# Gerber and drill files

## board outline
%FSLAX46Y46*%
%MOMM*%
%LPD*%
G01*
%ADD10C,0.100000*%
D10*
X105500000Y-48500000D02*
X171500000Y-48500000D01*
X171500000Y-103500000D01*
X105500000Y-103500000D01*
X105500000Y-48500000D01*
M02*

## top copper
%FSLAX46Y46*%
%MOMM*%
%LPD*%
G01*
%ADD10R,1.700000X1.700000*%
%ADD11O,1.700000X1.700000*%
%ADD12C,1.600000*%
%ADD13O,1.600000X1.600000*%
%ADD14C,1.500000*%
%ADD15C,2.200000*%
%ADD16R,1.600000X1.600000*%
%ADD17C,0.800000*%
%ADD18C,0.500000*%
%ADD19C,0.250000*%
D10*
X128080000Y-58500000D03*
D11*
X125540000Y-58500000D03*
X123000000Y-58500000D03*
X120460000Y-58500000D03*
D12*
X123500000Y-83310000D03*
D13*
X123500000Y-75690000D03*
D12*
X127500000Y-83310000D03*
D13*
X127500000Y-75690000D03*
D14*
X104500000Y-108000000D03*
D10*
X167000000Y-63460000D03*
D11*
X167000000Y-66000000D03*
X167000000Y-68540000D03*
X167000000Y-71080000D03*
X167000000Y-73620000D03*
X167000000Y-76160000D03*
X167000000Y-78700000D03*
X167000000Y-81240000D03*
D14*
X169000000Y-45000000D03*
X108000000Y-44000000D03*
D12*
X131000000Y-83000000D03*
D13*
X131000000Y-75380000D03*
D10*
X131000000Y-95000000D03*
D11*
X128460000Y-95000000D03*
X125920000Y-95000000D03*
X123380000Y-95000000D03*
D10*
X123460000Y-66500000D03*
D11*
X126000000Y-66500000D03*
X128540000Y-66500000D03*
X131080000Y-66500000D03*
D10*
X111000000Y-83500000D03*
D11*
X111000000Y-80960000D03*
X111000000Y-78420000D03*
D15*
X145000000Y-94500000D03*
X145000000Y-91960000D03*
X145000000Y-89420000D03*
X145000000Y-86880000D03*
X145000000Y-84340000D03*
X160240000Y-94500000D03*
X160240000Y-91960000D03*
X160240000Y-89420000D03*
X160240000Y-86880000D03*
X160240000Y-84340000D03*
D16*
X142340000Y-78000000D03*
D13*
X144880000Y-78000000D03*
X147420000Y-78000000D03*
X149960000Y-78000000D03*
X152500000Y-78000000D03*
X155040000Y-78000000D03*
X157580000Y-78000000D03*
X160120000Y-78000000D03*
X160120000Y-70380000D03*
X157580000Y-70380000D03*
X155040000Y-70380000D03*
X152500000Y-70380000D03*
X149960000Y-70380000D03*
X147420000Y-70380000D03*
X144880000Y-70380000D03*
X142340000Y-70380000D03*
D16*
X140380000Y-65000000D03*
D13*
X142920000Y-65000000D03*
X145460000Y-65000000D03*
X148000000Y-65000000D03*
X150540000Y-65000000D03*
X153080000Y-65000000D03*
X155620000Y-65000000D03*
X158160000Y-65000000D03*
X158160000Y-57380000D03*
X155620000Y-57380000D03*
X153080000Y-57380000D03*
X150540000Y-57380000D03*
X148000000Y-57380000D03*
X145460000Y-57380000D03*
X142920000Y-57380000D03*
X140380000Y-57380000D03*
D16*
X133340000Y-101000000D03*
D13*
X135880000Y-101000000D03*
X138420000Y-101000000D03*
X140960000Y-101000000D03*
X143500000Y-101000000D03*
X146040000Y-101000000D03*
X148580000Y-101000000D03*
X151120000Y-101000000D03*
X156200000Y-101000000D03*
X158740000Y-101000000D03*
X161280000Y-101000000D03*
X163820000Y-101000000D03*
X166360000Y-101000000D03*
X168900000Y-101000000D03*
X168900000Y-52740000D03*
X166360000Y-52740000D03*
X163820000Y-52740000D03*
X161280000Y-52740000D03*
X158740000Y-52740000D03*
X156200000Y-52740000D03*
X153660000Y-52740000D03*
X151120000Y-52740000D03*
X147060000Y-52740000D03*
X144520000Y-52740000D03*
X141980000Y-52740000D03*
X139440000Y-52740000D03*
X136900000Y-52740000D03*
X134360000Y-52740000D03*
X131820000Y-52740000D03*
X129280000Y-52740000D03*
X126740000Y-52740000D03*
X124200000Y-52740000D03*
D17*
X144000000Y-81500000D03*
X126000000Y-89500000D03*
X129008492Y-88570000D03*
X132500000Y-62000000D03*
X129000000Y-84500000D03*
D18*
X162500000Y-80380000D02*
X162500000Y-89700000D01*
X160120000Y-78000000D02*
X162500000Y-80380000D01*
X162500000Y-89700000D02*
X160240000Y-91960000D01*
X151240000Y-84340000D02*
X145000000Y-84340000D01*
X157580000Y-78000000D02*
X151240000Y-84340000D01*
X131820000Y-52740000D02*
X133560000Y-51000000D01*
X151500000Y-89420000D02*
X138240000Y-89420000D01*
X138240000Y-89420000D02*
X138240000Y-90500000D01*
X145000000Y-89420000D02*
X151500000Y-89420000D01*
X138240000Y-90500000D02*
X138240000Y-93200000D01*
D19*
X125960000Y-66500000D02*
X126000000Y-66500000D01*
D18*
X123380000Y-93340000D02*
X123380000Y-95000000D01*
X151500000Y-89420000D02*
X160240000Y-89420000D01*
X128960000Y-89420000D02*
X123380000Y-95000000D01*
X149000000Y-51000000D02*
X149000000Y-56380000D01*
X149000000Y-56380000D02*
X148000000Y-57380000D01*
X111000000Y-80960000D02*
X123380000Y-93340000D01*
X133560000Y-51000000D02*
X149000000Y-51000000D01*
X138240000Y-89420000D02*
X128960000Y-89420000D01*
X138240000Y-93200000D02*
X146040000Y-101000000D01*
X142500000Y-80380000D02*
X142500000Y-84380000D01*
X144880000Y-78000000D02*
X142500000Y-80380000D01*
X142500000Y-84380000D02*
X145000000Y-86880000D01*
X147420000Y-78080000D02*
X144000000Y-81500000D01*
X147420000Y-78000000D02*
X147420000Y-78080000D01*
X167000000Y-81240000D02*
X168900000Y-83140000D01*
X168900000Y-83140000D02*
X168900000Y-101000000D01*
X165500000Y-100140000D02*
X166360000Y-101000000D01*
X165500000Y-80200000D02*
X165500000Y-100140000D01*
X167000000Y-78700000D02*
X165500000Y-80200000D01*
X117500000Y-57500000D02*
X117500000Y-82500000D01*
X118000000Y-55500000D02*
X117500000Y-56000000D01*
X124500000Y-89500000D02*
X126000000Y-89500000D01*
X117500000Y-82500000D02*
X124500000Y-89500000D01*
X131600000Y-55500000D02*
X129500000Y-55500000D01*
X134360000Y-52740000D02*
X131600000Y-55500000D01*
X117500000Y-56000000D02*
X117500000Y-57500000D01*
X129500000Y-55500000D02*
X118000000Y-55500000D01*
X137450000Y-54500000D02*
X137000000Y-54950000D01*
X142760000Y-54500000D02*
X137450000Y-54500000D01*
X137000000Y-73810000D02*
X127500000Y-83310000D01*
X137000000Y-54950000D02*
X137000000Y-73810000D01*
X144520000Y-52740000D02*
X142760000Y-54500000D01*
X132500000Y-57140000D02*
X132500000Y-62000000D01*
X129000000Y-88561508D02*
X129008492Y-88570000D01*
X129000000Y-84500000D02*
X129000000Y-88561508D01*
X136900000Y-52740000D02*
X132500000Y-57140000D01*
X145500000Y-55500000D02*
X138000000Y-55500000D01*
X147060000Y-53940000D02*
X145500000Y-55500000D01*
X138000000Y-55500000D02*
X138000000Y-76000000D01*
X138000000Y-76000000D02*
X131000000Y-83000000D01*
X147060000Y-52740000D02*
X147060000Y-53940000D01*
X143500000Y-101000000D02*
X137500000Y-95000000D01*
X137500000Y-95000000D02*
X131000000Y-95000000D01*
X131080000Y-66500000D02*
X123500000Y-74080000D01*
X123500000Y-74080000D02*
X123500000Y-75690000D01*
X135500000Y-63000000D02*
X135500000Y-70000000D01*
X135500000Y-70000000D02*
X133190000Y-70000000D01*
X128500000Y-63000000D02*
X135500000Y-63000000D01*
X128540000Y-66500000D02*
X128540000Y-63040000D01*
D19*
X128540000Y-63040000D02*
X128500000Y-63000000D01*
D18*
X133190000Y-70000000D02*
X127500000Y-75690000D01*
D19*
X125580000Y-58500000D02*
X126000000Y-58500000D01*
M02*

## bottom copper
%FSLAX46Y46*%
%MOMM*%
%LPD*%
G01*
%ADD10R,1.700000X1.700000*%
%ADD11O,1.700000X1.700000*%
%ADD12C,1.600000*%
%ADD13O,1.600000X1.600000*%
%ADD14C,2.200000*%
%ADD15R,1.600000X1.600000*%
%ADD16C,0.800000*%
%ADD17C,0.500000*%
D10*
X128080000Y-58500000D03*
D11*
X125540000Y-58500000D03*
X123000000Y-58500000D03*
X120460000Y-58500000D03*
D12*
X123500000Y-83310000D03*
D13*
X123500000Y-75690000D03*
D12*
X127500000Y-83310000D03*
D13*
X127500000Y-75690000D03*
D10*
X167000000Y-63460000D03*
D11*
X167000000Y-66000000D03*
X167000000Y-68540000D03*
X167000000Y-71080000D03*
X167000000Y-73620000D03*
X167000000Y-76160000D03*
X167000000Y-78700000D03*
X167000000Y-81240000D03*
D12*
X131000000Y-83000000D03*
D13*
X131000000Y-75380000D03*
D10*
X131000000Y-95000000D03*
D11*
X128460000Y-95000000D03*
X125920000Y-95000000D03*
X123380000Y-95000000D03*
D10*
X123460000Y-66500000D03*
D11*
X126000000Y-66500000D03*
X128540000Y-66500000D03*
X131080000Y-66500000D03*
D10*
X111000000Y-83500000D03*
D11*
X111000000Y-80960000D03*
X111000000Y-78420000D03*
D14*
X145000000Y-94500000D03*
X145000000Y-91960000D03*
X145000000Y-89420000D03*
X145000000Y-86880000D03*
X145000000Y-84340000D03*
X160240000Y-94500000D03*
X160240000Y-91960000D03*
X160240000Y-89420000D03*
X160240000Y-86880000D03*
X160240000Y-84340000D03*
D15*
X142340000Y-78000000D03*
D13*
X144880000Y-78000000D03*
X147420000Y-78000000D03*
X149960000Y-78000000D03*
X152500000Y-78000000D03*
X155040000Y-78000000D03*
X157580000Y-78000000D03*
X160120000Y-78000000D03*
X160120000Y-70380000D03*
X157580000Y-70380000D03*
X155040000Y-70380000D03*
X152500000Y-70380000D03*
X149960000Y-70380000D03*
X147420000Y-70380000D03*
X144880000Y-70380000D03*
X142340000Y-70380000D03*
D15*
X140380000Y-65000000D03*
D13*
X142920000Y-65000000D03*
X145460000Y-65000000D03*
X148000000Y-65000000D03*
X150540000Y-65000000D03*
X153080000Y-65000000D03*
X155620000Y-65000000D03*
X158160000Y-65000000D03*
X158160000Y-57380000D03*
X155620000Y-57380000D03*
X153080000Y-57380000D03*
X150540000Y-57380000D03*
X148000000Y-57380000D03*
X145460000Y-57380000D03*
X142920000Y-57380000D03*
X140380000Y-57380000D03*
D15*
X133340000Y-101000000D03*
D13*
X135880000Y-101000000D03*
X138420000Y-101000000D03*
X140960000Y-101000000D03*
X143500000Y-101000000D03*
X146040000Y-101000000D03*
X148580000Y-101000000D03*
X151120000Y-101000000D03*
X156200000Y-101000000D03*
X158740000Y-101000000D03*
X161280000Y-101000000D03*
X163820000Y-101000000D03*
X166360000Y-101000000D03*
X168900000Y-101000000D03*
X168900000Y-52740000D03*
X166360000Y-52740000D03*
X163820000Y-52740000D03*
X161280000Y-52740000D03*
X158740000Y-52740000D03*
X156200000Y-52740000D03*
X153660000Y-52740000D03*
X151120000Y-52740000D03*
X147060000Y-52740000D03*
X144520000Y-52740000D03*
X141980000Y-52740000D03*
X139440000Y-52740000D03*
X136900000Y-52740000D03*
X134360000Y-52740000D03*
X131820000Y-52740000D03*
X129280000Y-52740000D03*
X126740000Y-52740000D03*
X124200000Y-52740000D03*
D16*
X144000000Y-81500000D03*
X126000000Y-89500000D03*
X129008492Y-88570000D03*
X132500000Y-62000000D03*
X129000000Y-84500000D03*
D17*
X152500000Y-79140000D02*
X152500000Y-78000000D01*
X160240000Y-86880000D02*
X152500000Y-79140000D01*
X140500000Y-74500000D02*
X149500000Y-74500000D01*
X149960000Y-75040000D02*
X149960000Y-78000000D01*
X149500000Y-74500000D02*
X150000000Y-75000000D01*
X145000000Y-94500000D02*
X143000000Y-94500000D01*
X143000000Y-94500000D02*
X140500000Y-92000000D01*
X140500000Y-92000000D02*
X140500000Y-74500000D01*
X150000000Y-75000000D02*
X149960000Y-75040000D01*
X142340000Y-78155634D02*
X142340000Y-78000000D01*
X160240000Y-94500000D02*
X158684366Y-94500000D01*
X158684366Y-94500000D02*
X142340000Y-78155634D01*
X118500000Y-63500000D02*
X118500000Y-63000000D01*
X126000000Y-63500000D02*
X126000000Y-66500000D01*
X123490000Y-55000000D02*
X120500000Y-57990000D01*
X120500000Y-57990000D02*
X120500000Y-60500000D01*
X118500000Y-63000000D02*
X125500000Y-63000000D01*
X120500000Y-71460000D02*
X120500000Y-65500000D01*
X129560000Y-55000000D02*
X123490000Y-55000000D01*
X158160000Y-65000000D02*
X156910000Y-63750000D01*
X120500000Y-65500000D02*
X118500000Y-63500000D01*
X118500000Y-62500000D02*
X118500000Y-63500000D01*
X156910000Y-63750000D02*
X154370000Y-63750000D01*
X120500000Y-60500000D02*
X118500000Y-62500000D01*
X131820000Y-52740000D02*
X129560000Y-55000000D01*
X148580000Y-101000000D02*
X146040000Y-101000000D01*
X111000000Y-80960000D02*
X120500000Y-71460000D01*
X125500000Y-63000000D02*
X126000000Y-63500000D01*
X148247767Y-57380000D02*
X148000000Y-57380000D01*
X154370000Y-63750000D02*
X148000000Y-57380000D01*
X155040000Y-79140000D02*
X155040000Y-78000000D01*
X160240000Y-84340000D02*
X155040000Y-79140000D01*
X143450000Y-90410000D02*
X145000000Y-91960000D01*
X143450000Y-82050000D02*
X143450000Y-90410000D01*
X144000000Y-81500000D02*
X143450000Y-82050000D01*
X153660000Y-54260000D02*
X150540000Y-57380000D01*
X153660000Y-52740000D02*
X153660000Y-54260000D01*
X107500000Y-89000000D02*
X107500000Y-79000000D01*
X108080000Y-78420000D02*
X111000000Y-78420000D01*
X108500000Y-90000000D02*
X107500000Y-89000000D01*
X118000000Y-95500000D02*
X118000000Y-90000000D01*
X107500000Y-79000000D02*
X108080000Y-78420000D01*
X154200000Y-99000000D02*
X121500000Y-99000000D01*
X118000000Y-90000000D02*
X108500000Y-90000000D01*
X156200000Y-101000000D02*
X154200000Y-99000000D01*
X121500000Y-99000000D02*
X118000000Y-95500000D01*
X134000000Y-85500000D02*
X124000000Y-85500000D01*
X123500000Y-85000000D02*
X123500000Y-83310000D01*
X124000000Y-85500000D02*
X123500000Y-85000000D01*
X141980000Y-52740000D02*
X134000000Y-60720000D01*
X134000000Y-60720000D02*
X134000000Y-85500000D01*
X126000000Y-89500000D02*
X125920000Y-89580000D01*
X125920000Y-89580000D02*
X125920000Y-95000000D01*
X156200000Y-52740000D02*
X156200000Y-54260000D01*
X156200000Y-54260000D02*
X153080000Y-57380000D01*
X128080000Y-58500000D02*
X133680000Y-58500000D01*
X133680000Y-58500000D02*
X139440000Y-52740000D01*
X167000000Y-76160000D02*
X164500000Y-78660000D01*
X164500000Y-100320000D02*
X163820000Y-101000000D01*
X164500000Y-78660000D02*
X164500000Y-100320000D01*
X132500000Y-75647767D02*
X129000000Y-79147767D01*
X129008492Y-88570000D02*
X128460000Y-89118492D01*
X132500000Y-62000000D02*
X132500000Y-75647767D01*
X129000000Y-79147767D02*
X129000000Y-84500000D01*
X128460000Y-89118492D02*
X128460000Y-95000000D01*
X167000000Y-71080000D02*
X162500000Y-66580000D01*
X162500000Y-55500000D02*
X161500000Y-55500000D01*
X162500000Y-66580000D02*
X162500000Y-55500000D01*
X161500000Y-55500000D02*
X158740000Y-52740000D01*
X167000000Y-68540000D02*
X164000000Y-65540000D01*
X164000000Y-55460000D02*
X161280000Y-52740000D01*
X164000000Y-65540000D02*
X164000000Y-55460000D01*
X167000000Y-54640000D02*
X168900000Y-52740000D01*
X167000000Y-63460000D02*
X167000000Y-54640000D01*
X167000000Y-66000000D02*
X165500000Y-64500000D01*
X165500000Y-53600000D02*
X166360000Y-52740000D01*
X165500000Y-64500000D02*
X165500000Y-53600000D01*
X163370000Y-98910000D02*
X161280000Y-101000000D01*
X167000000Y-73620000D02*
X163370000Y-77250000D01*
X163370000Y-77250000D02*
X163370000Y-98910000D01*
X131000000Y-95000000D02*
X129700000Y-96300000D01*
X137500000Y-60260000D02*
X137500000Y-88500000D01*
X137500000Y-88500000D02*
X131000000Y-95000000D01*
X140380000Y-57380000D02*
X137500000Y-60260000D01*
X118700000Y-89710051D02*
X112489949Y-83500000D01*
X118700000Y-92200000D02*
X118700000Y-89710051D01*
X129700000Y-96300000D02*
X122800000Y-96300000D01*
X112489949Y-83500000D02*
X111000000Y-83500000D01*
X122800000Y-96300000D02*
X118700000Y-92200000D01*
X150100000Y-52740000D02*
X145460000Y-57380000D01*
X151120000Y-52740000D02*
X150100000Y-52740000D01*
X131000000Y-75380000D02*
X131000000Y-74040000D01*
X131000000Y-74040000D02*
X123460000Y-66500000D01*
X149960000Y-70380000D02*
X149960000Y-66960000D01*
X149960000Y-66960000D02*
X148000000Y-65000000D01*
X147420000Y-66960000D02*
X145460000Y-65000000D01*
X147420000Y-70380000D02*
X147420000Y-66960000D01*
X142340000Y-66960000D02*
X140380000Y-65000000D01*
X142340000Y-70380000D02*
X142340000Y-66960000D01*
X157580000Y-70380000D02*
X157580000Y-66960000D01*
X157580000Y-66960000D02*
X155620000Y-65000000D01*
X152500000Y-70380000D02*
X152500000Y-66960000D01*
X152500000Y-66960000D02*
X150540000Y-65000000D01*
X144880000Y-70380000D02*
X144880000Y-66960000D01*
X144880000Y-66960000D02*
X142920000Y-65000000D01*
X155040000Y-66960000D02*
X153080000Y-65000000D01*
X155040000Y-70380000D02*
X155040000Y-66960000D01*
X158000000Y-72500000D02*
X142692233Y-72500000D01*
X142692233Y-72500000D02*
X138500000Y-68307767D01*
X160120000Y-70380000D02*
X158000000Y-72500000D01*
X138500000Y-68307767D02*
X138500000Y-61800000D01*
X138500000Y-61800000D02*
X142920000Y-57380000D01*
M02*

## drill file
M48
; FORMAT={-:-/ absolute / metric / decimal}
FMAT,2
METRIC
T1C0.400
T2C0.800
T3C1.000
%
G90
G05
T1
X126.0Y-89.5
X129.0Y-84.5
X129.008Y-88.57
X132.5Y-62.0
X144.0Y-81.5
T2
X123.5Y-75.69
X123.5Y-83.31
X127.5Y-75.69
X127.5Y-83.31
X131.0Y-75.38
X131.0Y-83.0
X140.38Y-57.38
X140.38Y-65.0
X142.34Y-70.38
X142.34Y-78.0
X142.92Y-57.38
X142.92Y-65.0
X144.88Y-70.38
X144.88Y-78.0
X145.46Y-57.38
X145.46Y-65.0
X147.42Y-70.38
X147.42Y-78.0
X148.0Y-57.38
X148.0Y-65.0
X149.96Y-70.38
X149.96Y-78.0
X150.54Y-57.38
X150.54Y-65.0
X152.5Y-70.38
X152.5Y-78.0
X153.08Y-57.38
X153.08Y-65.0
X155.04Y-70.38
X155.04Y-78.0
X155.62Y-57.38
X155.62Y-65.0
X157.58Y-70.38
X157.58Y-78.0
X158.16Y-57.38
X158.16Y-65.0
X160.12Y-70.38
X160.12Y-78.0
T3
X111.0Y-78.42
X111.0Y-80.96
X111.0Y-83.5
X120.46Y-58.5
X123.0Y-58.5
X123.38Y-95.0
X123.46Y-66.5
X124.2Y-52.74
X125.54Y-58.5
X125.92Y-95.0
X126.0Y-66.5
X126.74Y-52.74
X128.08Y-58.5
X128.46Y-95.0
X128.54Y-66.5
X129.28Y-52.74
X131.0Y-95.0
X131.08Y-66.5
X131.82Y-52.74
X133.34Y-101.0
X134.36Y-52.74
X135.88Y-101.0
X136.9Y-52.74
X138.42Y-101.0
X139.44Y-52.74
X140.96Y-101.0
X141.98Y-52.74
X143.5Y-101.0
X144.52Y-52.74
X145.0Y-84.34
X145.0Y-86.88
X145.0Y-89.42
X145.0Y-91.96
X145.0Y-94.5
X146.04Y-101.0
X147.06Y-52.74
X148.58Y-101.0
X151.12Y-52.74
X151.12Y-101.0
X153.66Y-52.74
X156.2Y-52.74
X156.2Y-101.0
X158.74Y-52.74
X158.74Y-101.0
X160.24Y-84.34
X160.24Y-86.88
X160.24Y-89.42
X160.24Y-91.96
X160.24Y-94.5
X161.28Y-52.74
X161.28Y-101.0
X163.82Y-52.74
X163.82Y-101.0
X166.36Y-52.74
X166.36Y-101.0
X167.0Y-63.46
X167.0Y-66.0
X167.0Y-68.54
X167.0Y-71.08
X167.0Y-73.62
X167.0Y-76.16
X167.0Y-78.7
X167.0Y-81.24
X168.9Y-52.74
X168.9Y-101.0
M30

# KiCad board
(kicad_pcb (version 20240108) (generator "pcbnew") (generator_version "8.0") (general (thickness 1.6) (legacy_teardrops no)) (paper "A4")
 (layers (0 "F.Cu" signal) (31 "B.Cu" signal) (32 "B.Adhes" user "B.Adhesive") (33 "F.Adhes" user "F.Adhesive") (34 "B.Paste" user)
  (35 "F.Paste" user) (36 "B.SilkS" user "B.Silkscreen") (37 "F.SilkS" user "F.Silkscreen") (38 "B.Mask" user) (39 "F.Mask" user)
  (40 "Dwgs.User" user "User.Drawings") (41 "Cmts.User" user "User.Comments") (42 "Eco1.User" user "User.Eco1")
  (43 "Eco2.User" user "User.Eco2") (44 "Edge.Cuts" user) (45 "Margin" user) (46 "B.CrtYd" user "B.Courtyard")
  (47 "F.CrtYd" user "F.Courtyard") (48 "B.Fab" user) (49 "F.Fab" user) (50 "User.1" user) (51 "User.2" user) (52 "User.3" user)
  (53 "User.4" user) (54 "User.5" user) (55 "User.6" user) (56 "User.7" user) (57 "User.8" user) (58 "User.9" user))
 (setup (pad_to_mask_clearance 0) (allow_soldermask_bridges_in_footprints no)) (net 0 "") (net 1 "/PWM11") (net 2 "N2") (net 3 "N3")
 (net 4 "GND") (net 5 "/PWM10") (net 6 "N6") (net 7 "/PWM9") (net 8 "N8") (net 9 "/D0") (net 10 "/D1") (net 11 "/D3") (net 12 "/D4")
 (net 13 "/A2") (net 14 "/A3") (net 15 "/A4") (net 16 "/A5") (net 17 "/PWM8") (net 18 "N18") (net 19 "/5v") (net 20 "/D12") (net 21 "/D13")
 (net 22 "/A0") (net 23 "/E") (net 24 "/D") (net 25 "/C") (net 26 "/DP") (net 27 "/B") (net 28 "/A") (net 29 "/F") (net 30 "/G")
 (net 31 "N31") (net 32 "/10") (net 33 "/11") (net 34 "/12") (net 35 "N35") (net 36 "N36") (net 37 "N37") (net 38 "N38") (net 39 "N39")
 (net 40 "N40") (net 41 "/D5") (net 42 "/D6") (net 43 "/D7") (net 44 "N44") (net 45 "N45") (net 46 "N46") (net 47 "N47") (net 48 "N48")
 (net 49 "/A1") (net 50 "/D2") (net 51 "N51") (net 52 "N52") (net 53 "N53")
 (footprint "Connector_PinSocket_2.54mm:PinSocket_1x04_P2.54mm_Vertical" (layer "F.Cu") (at 128.08 58.5 -90)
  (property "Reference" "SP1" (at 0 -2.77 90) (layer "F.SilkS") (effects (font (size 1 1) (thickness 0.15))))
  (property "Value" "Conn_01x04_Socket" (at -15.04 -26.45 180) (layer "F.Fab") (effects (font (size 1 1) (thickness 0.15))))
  (pad "1" thru_hole rect (at 0 0 270) (size 1.7 1.7) (drill 1) (layers "*.Cu" "*.Mask") (remove_unused_layers no) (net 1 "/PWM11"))
  (pad "2" thru_hole oval (at 0 2.54 270) (size 1.7 1.7) (drill 1) (layers "*.Cu" "*.Mask") (remove_unused_layers no) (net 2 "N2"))
  (pad "3" thru_hole oval (at 0 5.08 270) (size 1.7 1.7) (drill 1) (layers "*.Cu" "*.Mask") (remove_unused_layers no) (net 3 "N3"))
  (pad "4" thru_hole oval (at 0 7.62 270) (size 1.7 1.7) (drill 1) (layers "*.Cu" "*.Mask") (remove_unused_layers no) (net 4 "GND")))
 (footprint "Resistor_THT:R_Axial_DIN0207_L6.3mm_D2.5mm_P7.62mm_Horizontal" (layer "F.Cu") (at 123.5 83.31 90)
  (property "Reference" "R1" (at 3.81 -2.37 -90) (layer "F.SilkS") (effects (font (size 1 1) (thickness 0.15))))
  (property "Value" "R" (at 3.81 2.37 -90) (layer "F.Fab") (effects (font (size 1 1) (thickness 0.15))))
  (pad "1" thru_hole circle (at 0 0 90) (size 1.6 1.6) (drill 0.8) (layers "*.Cu" "*.Mask") (remove_unused_layers no) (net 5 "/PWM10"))
  (pad "2" thru_hole oval (at 7.62 0 90) (size 1.6 1.6) (drill 0.8) (layers "*.Cu" "*.Mask") (remove_unused_layers no) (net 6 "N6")))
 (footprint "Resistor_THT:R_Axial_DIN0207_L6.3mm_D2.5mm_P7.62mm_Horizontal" (layer "F.Cu") (at 127.5 83.31 90)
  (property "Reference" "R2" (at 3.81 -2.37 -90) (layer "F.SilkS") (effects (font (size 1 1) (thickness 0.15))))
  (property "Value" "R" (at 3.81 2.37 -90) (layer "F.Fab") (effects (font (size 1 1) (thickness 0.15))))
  (pad "1" thru_hole circle (at 0 0 90) (size 1.6 1.6) (drill 0.8) (layers "*.Cu" "*.Mask") (remove_unused_layers no) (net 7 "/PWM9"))
  (pad "2" thru_hole oval (at 7.62 0 90) (size 1.6 1.6) (drill 0.8) (layers "*.Cu" "*.Mask") (remove_unused_layers no) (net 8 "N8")))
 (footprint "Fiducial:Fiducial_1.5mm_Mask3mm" (layer "F.Cu") (at 104.5 108)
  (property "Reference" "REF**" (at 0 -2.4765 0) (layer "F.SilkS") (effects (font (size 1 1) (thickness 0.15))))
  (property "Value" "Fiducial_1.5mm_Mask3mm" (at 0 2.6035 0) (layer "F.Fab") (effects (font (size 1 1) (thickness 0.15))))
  (pad "" smd circle (at 0 0) (size 1.5 1.5) (layers "F.Cu" "F.Mask") (solder_mask_margin 0.75) (clearance 0.75)))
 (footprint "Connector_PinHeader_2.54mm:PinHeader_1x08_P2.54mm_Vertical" (layer "F.Cu") (at 167 63.46)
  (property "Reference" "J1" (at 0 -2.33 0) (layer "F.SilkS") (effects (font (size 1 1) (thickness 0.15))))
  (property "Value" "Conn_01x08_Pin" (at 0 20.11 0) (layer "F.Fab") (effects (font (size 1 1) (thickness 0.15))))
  (pad "1" thru_hole rect (at 0 0) (size 1.7 1.7) (drill 1) (layers "*.Cu" "*.Mask") (remove_unused_layers no) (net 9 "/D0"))
  (pad "2" thru_hole oval (at 0 2.54) (size 1.7 1.7) (drill 1) (layers "*.Cu" "*.Mask") (remove_unused_layers no) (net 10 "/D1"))
  (pad "3" thru_hole oval (at 0 5.08) (size 1.7 1.7) (drill 1) (layers "*.Cu" "*.Mask") (remove_unused_layers no) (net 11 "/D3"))
  (pad "4" thru_hole oval (at 0 7.62) (size 1.7 1.7) (drill 1) (layers "*.Cu" "*.Mask") (remove_unused_layers no) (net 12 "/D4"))
  (pad "5" thru_hole oval (at 0 10.16) (size 1.7 1.7) (drill 1) (layers "*.Cu" "*.Mask") (remove_unused_layers no) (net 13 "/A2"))
  (pad "6" thru_hole oval (at 0 12.7) (size 1.7 1.7) (drill 1) (layers "*.Cu" "*.Mask") (remove_unused_layers no) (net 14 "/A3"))
  (pad "7" thru_hole oval (at 0 15.24) (size 1.7 1.7) (drill 1) (layers "*.Cu" "*.Mask") (remove_unused_layers no) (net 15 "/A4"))
  (pad "8" thru_hole oval (at 0 17.78) (size 1.7 1.7) (drill 1) (layers "*.Cu" "*.Mask") (remove_unused_layers no) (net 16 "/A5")))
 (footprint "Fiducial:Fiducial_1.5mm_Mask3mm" (layer "F.Cu") (at 169 45)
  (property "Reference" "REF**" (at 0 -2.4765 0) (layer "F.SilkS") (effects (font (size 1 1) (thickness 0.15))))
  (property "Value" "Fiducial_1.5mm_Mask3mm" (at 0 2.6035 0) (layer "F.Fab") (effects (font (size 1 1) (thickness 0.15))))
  (pad "" smd circle (at 0 0) (size 1.5 1.5) (layers "F.Cu" "F.Mask") (solder_mask_margin 0.75) (clearance 0.75)))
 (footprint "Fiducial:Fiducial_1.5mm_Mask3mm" (layer "F.Cu") (at 108 44)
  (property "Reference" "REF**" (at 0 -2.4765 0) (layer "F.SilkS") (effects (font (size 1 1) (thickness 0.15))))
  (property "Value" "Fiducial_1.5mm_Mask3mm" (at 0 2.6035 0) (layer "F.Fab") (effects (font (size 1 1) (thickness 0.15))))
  (pad "" smd circle (at 0 0) (size 1.5 1.5) (layers "F.Cu" "F.Mask") (solder_mask_margin 0.75) (clearance 0.75)))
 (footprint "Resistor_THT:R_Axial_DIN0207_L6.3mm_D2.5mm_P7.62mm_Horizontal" (layer "F.Cu") (at 131 83 90)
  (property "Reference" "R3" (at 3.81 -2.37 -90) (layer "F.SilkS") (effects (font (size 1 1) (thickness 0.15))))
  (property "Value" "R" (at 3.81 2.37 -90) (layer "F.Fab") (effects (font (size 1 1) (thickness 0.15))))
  (pad "1" thru_hole circle (at 0 0 90) (size 1.6 1.6) (drill 0.8) (layers "*.Cu" "*.Mask") (remove_unused_layers no) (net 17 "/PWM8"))
  (pad "2" thru_hole oval (at 7.62 0 90) (size 1.6 1.6) (drill 0.8) (layers "*.Cu" "*.Mask") (remove_unused_layers no) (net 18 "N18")))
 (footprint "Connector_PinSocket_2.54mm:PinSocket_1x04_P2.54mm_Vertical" (layer "F.Cu") (at 131 95 -90)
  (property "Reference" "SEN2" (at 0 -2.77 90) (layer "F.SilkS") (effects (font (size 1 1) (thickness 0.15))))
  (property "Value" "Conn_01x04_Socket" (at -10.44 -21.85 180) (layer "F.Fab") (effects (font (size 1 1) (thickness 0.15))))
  (pad "1" thru_hole rect (at 0 0 270) (size 1.7 1.7) (drill 1) (layers "*.Cu" "*.Mask") (remove_unused_layers no) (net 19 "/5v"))
  (pad "2" thru_hole oval (at 0 2.54 270) (size 1.7 1.7) (drill 1) (layers "*.Cu" "*.Mask") (remove_unused_layers no) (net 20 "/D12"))
  (pad "3" thru_hole oval (at 0 5.08 270) (size 1.7 1.7) (drill 1) (layers "*.Cu" "*.Mask") (remove_unused_layers no) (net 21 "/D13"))
  (pad "4" thru_hole oval (at 0 7.62 270) (size 1.7 1.7) (drill 1) (layers "*.Cu" "*.Mask") (remove_unused_layers no) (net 4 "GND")))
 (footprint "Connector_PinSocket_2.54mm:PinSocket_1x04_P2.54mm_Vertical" (layer "F.Cu") (at 123.46 66.5 90)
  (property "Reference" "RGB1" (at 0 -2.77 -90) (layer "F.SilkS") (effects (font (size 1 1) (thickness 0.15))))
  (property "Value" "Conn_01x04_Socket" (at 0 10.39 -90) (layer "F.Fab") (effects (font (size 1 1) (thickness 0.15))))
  (pad "1" thru_hole rect (at 0 0 90) (size 1.7 1.7) (drill 1) (layers "*.Cu" "*.Mask") (remove_unused_layers no) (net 18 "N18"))
  (pad "2" thru_hole oval (at 0 2.54 90) (size 1.7 1.7) (drill 1) (layers "*.Cu" "*.Mask") (remove_unused_layers no) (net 4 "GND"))
  (pad "3" thru_hole oval (at 0 5.08 90) (size 1.7 1.7) (drill 1) (layers "*.Cu" "*.Mask") (remove_unused_layers no) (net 8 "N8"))
  (pad "4" thru_hole oval (at 0 7.62 90) (size 1.7 1.7) (drill 1) (layers "*.Cu" "*.Mask") (remove_unused_layers no) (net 6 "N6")))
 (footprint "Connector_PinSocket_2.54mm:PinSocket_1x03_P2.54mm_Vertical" (layer "F.Cu") (at 111 83.5 180)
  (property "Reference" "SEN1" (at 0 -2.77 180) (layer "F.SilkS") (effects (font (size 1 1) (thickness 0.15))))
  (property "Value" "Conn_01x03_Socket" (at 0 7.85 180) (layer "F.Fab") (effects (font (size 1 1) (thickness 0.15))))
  (pad "1" thru_hole rect (at 0 0 180) (size 1.7 1.7) (drill 1) (layers "*.Cu" "*.Mask") (remove_unused_layers no) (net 19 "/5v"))
  (pad "2" thru_hole oval (at 0 2.54 180) (size 1.7 1.7) (drill 1) (layers "*.Cu" "*.Mask") (remove_unused_layers no) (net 4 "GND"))
  (pad "3" thru_hole oval (at 0 5.08 180) (size 1.7 1.7) (drill 1) (layers "*.Cu" "*.Mask") (remove_unused_layers no) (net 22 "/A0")))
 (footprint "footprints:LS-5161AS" (layer "F.Cu") (at 145 94.5 90)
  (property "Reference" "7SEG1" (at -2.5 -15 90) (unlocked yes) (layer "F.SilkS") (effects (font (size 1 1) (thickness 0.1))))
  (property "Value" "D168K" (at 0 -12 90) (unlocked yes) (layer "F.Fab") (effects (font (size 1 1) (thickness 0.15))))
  (pad "1" thru_hole circle (at 0 0 90) (size 2.2 2.2) (drill 1) (layers "*.Cu" "*.Mask") (remove_unused_layers no) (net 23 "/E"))
  (pad "2" thru_hole circle (at 2.54 0 90) (size 2.2 2.2) (drill 1) (layers "*.Cu" "*.Mask") (remove_unused_layers no) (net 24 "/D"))
  (pad "3" thru_hole circle (at 5.08 0 90) (size 2.2 2.2) (drill 1) (layers "*.Cu" "*.Mask") (remove_unused_layers no) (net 4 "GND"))
  (pad "4" thru_hole circle (at 7.62 0 90) (size 2.2 2.2) (drill 1) (layers "*.Cu" "*.Mask") (remove_unused_layers no) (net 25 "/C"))
  (pad "5" thru_hole circle (at 10.16 0 90) (size 2.2 2.2) (drill 1) (layers "*.Cu" "*.Mask") (remove_unused_layers no) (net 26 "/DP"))
  (pad "6" thru_hole circle (at 0 15.24 90) (size 2.2 2.2) (drill 1) (layers "*.Cu" "*.Mask") (remove_unused_layers no) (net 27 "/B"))
  (pad "7" thru_hole circle (at 2.54 15.24 90) (size 2.2 2.2) (drill 1) (layers "*.Cu" "*.Mask") (remove_unused_layers no) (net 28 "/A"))
  (pad "8" thru_hole circle (at 5.08 15.24 90) (size 2.2 2.2) (drill 1) (layers "*.Cu" "*.Mask") (remove_unused_layers no) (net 4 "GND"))
  (pad "9" thru_hole circle (at 7.62 15.24 90) (size 2.2 2.2) (drill 1) (layers "*.Cu" "*.Mask") (remove_unused_layers no) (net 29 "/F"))
  (pad "10" thru_hole circle (at 10.16 15.24 90) (size 2.2 2.2) (drill 1) (layers "*.Cu" "*.Mask") (remove_unused_layers no) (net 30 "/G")))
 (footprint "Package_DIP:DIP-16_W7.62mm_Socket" (layer "F.Cu") (at 142.34 78 90)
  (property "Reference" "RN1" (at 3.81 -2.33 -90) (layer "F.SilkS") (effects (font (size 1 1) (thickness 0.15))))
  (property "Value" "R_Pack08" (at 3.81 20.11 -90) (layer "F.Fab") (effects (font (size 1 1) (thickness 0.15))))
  (pad "1" thru_hole rect (at 0 0 90) (size 1.6 1.6) (drill 0.8) (layers "*.Cu" "*.Mask") (remove_unused_layers no) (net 27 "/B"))
  (pad "2" thru_hole oval (at 0 2.54 90) (size 1.6 1.6) (drill 0.8) (layers "*.Cu" "*.Mask") (remove_unused_layers no) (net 25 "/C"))
  (pad "3" thru_hole oval (at 0 5.08 90) (size 1.6 1.6) (drill 0.8) (layers "*.Cu" "*.Mask") (remove_unused_layers no) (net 24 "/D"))
  (pad "4" thru_hole oval (at 0 7.62 90) (size 1.6 1.6) (drill 0.8) (layers "*.Cu" "*.Mask") (remove_unused_layers no) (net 23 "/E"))
  (pad "5" thru_hole oval (at 0 10.16 90) (size 1.6 1.6) (drill 0.8) (layers "*.Cu" "*.Mask") (remove_unused_layers no) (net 29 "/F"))
  (pad "6" thru_hole oval (at 0 12.7 90) (size 1.6 1.6) (drill 0.8) (layers "*.Cu" "*.Mask") (remove_unused_layers no) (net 30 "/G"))
  (pad "7" thru_hole oval (at 0 15.24 90) (size 1.6 1.6) (drill 0.8) (layers "*.Cu" "*.Mask") (remove_unused_layers no) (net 26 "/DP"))
  (pad "8" thru_hole oval (at 0 17.78 90) (size 1.6 1.6) (drill 0.8) (layers "*.Cu" "*.Mask") (remove_unused_layers no) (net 28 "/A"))
  (pad "9" thru_hole oval (at 7.62 17.78 90) (size 1.6 1.6) (drill 0.8) (layers "*.Cu" "*.Mask") (remove_unused_layers no) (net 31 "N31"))
  (pad "10" thru_hole oval (at 7.62 15.24 90) (size 1.6 1.6) (drill 0.8) (layers "*.Cu" "*.Mask") (remove_unused_layers no) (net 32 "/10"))
  (pad "11" thru_hole oval (at 7.62 12.7 90) (size 1.6 1.6) (drill 0.8) (layers "*.Cu" "*.Mask") (remove_unused_layers no) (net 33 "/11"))
  (pad "12" thru_hole oval (at 7.62 10.16 90) (size 1.6 1.6) (drill 0.8) (layers "*.Cu" "*.Mask") (remove_unused_layers no) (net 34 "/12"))
  (pad "13" thru_hole oval (at 7.62 7.62 90) (size 1.6 1.6) (drill 0.8) (layers "*.Cu" "*.Mask") (remove_unused_layers no) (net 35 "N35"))
  (pad "14" thru_hole oval (at 7.62 5.08 90) (size 1.6 1.6) (drill 0.8) (layers "*.Cu" "*.Mask") (remove_unused_layers no) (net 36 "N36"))
  (pad "15" thru_hole oval (at 7.62 2.54 90) (size 1.6 1.6) (drill 0.8) (layers "*.Cu" "*.Mask") (remove_unused_layers no) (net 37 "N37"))
  (pad "16" thru_hole oval (at 7.62 0 90) (size 1.6 1.6) (drill 0.8) (layers "*.Cu" "*.Mask") (remove_unused_layers no) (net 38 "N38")))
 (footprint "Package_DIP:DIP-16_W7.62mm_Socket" (layer "F.Cu") (at 140.38 65 90)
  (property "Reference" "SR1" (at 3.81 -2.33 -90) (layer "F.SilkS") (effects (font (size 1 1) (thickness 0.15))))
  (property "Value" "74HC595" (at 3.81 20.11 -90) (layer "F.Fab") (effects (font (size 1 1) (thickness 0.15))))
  (pad "1" thru_hole rect (at 0 0 90) (size 1.6 1.6) (drill 0.8) (layers "*.Cu" "*.Mask") (remove_unused_layers no) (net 38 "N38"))
  (pad "2" thru_hole oval (at 0 2.54 90) (size 1.6 1.6) (drill 0.8) (layers "*.Cu" "*.Mask") (remove_unused_layers no) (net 37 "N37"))
  (pad "3" thru_hole oval (at 0 5.08 90) (size 1.6 1.6) (drill 0.8) (layers "*.Cu" "*.Mask") (remove_unused_layers no) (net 36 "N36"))
  (pad "4" thru_hole oval (at 0 7.62 90) (size 1.6 1.6) (drill 0.8) (layers "*.Cu" "*.Mask") (remove_unused_layers no) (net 35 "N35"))
  (pad "5" thru_hole oval (at 0 10.16 90) (size 1.6 1.6) (drill 0.8) (layers "*.Cu" "*.Mask") (remove_unused_layers no) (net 34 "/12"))
  (pad "6" thru_hole oval (at 0 12.7 90) (size 1.6 1.6) (drill 0.8) (layers "*.Cu" "*.Mask") (remove_unused_layers no) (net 33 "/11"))
  (pad "7" thru_hole oval (at 0 15.24 90) (size 1.6 1.6) (drill 0.8) (layers "*.Cu" "*.Mask") (remove_unused_layers no) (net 32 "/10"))
  (pad "8" thru_hole oval (at 0 17.78 90) (size 1.6 1.6) (drill 0.8) (layers "*.Cu" "*.Mask") (remove_unused_layers no) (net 4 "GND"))
  (pad "9" thru_hole oval (at 7.62 17.78 90) (size 1.6 1.6) (drill 0.8) (layers "*.Cu" "*.Mask") (remove_unused_layers no) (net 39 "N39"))
  (pad "10" thru_hole oval (at 7.62 15.24 90) (size 1.6 1.6) (drill 0.8) (layers "*.Cu" "*.Mask") (remove_unused_layers no) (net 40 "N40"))
  (pad "11" thru_hole oval (at 7.62 12.7 90) (size 1.6 1.6) (drill 0.8) (layers "*.Cu" "*.Mask") (remove_unused_layers no) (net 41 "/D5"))
  (pad "12" thru_hole oval (at 7.62 10.16 90) (size 1.6 1.6) (drill 0.8) (layers "*.Cu" "*.Mask") (remove_unused_layers no) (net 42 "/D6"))
  (pad "13" thru_hole oval (at 7.62 7.62 90) (size 1.6 1.6) (drill 0.8) (layers "*.Cu" "*.Mask") (remove_unused_layers no) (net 4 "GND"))
  (pad "14" thru_hole oval (at 7.62 5.08 90) (size 1.6 1.6) (drill 0.8) (layers "*.Cu" "*.Mask") (remove_unused_layers no) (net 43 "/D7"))
  (pad "15" thru_hole oval (at 7.62 2.54 90) (size 1.6 1.6) (drill 0.8) (layers "*.Cu" "*.Mask") (remove_unused_layers no) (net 31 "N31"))
  (pad "16" thru_hole oval (at 7.62 0 90) (size 1.6 1.6) (drill 0.8) (layers "*.Cu" "*.Mask") (remove_unused_layers no) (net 19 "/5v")))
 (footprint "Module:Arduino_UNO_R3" (layer "B.Cu") (at 133.34 101)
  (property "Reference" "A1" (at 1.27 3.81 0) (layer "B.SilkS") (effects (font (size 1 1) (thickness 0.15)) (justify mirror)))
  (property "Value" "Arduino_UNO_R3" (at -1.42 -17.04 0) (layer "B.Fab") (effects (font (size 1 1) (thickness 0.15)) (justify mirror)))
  (pad "1" thru_hole rect (at 0 0 270) (size 1.6 1.6) (drill 1) (layers "*.Cu" "*.Mask") (remove_unused_layers no) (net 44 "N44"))
  (pad "2" thru_hole oval (at 2.54 0 270) (size 1.6 1.6) (drill 1) (layers "*.Cu" "*.Mask") (remove_unused_layers no) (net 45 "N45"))
  (pad "3" thru_hole oval (at 5.08 0 270) (size 1.6 1.6) (drill 1) (layers "*.Cu" "*.Mask") (remove_unused_layers no) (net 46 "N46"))
  (pad "4" thru_hole oval (at 7.62 0 270) (size 1.6 1.6) (drill 1) (layers "*.Cu" "*.Mask") (remove_unused_layers no) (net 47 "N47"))
  (pad "5" thru_hole oval (at 10.16 0 270) (size 1.6 1.6) (drill 1) (layers "*.Cu" "*.Mask") (remove_unused_layers no) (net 19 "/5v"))
  (pad "6" thru_hole oval (at 12.7 0 270) (size 1.6 1.6) (drill 1) (layers "*.Cu" "*.Mask") (remove_unused_layers no) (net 4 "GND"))
  (pad "7" thru_hole oval (at 15.24 0 270) (size 1.6 1.6) (drill 1) (layers "*.Cu" "*.Mask") (remove_unused_layers no) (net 4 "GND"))
  (pad "8" thru_hole oval (at 17.78 0 270) (size 1.6 1.6) (drill 1) (layers "*.Cu" "*.Mask") (remove_unused_layers no) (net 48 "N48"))
  (pad "9" thru_hole oval (at 22.86 0 270) (size 1.6 1.6) (drill 1) (layers "*.Cu" "*.Mask") (remove_unused_layers no) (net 22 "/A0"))
  (pad "10" thru_hole oval (at 25.4 0 270) (size 1.6 1.6) (drill 1) (layers "*.Cu" "*.Mask") (remove_unused_layers no) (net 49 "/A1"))
  (pad "11" thru_hole oval (at 27.94 0 270) (size 1.6 1.6) (drill 1) (layers "*.Cu" "*.Mask") (remove_unused_layers no) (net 13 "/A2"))
  (pad "12" thru_hole oval (at 30.48 0 270) (size 1.6 1.6) (drill 1) (layers "*.Cu" "*.Mask") (remove_unused_layers no) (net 14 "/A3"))
  (pad "13" thru_hole oval (at 33.02 0 270) (size 1.6 1.6) (drill 1) (layers "*.Cu" "*.Mask") (remove_unused_layers no) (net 15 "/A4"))
  (pad "14" thru_hole oval (at 35.56 0 270) (size 1.6 1.6) (drill 1) (layers "*.Cu" "*.Mask") (remove_unused_layers no) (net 16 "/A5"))
  (pad "15" thru_hole oval (at 35.56 -48.26 270) (size 1.6 1.6) (drill 1) (layers "*.Cu" "*.Mask") (remove_unused_layers no) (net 9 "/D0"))
  (pad "16" thru_hole oval (at 33.02 -48.26 270) (size 1.6 1.6) (drill 1) (layers "*.Cu" "*.Mask") (remove_unused_layers no) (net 10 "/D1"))
  (pad "17" thru_hole oval (at 30.48 -48.26 270) (size 1.6 1.6) (drill 1) (layers "*.Cu" "*.Mask") (remove_unused_layers no) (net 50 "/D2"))
  (pad "18" thru_hole oval (at 27.94 -48.26 270) (size 1.6 1.6) (drill 1) (layers "*.Cu" "*.Mask") (remove_unused_layers no) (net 11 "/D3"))
  (pad "19" thru_hole oval (at 25.4 -48.26 270) (size 1.6 1.6) (drill 1) (layers "*.Cu" "*.Mask") (remove_unused_layers no) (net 12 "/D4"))
  (pad "20" thru_hole oval (at 22.86 -48.26 270) (size 1.6 1.6) (drill 1) (layers "*.Cu" "*.Mask") (remove_unused_layers no) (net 41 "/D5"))
  (pad "21" thru_hole oval (at 20.32 -48.26 270) (size 1.6 1.6) (drill 1) (layers "*.Cu" "*.Mask") (remove_unused_layers no) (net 42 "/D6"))
  (pad "22" thru_hole oval (at 17.78 -48.26 270) (size 1.6 1.6) (drill 1) (layers "*.Cu" "*.Mask") (remove_unused_layers no) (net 43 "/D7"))
  (pad "23" thru_hole oval (at 13.72 -48.26 270) (size 1.6 1.6) (drill 1) (layers "*.Cu" "*.Mask") (remove_unused_layers no)
   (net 17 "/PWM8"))
  (pad "24" thru_hole oval (at 11.18 -48.26 270) (size 1.6 1.6) (drill 1) (layers "*.Cu" "*.Mask") (remove_unused_layers no) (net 7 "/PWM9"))
  (pad "25" thru_hole oval (at 8.64 -48.26 270) (size 1.6 1.6) (drill 1) (layers "*.Cu" "*.Mask") (remove_unused_layers no) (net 5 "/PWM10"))
  (pad "26" thru_hole oval (at 6.1 -48.26 270) (size 1.6 1.6) (drill 1) (layers "*.Cu" "*.Mask") (remove_unused_layers no) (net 1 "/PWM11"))
  (pad "27" thru_hole oval (at 3.56 -48.26 270) (size 1.6 1.6) (drill 1) (layers "*.Cu" "*.Mask") (remove_unused_layers no) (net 20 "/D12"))
  (pad "28" thru_hole oval (at 1.02 -48.26 270) (size 1.6 1.6) (drill 1) (layers "*.Cu" "*.Mask") (remove_unused_layers no) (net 21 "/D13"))
  (pad "29" thru_hole oval (at -1.52 -48.26 270) (size 1.6 1.6) (drill 1) (layers "*.Cu" "*.Mask") (remove_unused_layers no) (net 4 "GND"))
  (pad "30" thru_hole oval (at -4.06 -48.26 270) (size 1.6 1.6) (drill 1) (layers "*.Cu" "*.Mask") (remove_unused_layers no) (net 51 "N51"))
  (pad "31" thru_hole oval (at -6.6 -48.26 270) (size 1.6 1.6) (drill 1) (layers "*.Cu" "*.Mask") (remove_unused_layers no) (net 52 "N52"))
  (pad "32" thru_hole oval (at -9.14 -48.26 270) (size 1.6 1.6) (drill 1) (layers "*.Cu" "*.Mask") (remove_unused_layers no) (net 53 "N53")))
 (gr_rect (start 105.5 48.5) (end 171.5 103.5) (stroke (width 0.1) (type default)) (fill none) (layer "Edge.Cuts"))
 (segment (start 152.5 79.14) (end 152.5 78) (width 0.5) (layer "B.Cu") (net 29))
 (segment (start 160.24 86.88) (end 152.5 79.14) (width 0.5) (layer "B.Cu") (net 29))
 (segment (start 162.5 80.38) (end 162.5 89.7) (width 0.5) (layer "F.Cu") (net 28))
 (segment (start 160.12 78) (end 162.5 80.38) (width 0.5) (layer "F.Cu") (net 28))
 (segment (start 162.5 89.7) (end 160.24 91.96) (width 0.5) (layer "F.Cu") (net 28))
 (segment (start 140.5 74.5) (end 149.5 74.5) (width 0.5) (layer "B.Cu") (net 23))
 (segment (start 149.96 75.04) (end 149.96 78) (width 0.5) (layer "B.Cu") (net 23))
 (segment (start 149.5 74.5) (end 150 75) (width 0.5) (layer "B.Cu") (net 23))
 (segment (start 145 94.5) (end 143 94.5) (width 0.5) (layer "B.Cu") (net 23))
 (segment (start 143 94.5) (end 140.5 92) (width 0.5) (layer "B.Cu") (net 23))
 (segment (start 140.5 92) (end 140.5 74.5) (width 0.5) (layer "B.Cu") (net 23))
 (segment (start 150 75) (end 149.96 75.04) (width 0.5) (layer "B.Cu") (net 23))
 (segment (start 151.24 84.34) (end 145 84.34) (width 0.5) (layer "F.Cu") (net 26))
 (segment (start 157.58 78) (end 151.24 84.34) (width 0.5) (layer "F.Cu") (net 26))
 (segment (start 142.34 78.155634) (end 142.34 78) (width 0.5) (layer "B.Cu") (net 27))
 (segment (start 160.24 94.5) (end 158.684366 94.5) (width 0.5) (layer "B.Cu") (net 27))
 (segment (start 158.684366 94.5) (end 142.34 78.155634) (width 0.5) (layer "B.Cu") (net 27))
 (segment (start 131.82 52.74) (end 133.56 51) (width 0.5) (layer "F.Cu") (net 4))
 (segment (start 151.5 89.42) (end 138.24 89.42) (width 0.5) (layer "F.Cu") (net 4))
 (segment (start 138.24 89.42) (end 138.24 90.5) (width 0.5) (layer "F.Cu") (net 4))
 (segment (start 145 89.42) (end 151.5 89.42) (width 0.5) (layer "F.Cu") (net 4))
 (segment (start 138.24 90.5) (end 138.24 93.2) (width 0.5) (layer "F.Cu") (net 4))
 (segment (start 125.96 66.5) (end 126 66.5) (width 0.25) (layer "F.Cu") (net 4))
 (segment (start 123.38 93.34) (end 123.38 95) (width 0.5) (layer "F.Cu") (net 4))
 (segment (start 151.5 89.42) (end 160.24 89.42) (width 0.5) (layer "F.Cu") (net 4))
 (segment (start 128.96 89.42) (end 123.38 95) (width 0.5) (layer "F.Cu") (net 4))
 (segment (start 149 51) (end 149 56.38) (width 0.5) (layer "F.Cu") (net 4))
 (segment (start 149 56.38) (end 148 57.38) (width 0.5) (layer "F.Cu") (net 4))
 (segment (start 111 80.96) (end 123.38 93.34) (width 0.5) (layer "F.Cu") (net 4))
 (segment (start 133.56 51) (end 149 51) (width 0.5) (layer "F.Cu") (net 4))
 (segment (start 138.24 89.42) (end 128.96 89.42) (width 0.5) (layer "F.Cu") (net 4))
 (segment (start 138.24 93.2) (end 146.04 101) (width 0.5) (layer "F.Cu") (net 4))
 (segment (start 118.5 63.5) (end 118.5 63) (width 0.5) (layer "B.Cu") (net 4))
 (segment (start 126 63.5) (end 126 66.5) (width 0.5) (layer "B.Cu") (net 4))
 (segment (start 123.49 55) (end 120.5 57.99) (width 0.5) (layer "B.Cu") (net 4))
 (segment (start 120.5 57.99) (end 120.5 60.5) (width 0.5) (layer "B.Cu") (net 4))
 (segment (start 118.5 63) (end 125.5 63) (width 0.5) (layer "B.Cu") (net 4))
 (segment (start 120.5 71.46) (end 120.5 65.5) (width 0.5) (layer "B.Cu") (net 4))
 (segment (start 129.56 55) (end 123.49 55) (width 0.5) (layer "B.Cu") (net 4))
 (segment (start 158.16 65) (end 156.91 63.75) (width 0.5) (layer "B.Cu") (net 4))
 (segment (start 120.5 65.5) (end 118.5 63.5) (width 0.5) (layer "B.Cu") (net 4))
 (segment (start 118.5 62.5) (end 118.5 63.5) (width 0.5) (layer "B.Cu") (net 4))
 (segment (start 156.91 63.75) (end 154.37 63.75) (width 0.5) (layer "B.Cu") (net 4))
 (segment (start 120.5 60.5) (end 118.5 62.5) (width 0.5) (layer "B.Cu") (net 4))
 (segment (start 131.82 52.74) (end 129.56 55) (width 0.5) (layer "B.Cu") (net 4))
 (segment (start 148.58 101) (end 146.04 101) (width 0.5) (layer "B.Cu") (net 4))
 (segment (start 111 80.96) (end 120.5 71.46) (width 0.5) (layer "B.Cu") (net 4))
 (segment (start 125.5 63) (end 126 63.5) (width 0.5) (layer "B.Cu") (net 4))
 (segment (start 148.247767 57.38) (end 148 57.38) (width 0.5) (layer "B.Cu") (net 4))
 (segment (start 154.37 63.75) (end 148 57.38) (width 0.5) (layer "B.Cu") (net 4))
 (segment (start 142.5 80.38) (end 142.5 84.38) (width 0.5) (layer "F.Cu") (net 25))
 (segment (start 144.88 78) (end 142.5 80.38) (width 0.5) (layer "F.Cu") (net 25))
 (segment (start 142.5 84.38) (end 145 86.88) (width 0.5) (layer "F.Cu") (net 25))
 (segment (start 155.04 79.14) (end 155.04 78) (width 0.5) (layer "B.Cu") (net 30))
 (segment (start 160.24 84.34) (end 155.04 79.14) (width 0.5) (layer "B.Cu") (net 30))
 (segment (start 147.42 78.08) (end 144 81.5) (width 0.5) (layer "F.Cu") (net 24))
 (segment (start 147.42 78) (end 147.42 78.08) (width 0.5) (layer "F.Cu") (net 24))
 (via (at 144 81.5) (size 0.8) (drill 0.4) (layers "F.Cu" "B.Cu") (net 24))
 (segment (start 143.45 90.41) (end 145 91.96) (width 0.5) (layer "B.Cu") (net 24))
 (segment (start 143.45 82.05) (end 143.45 90.41) (width 0.5) (layer "B.Cu") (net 24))
 (segment (start 144 81.5) (end 143.45 82.05) (width 0.5) (layer "B.Cu") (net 24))
 (segment (start 167 81.24) (end 168.9 83.14) (width 0.5) (layer "F.Cu") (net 16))
 (segment (start 168.9 83.14) (end 168.9 101) (width 0.5) (layer "F.Cu") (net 16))
 (segment (start 153.66 54.26) (end 150.54 57.38) (width 0.5) (layer "B.Cu") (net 42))
 (segment (start 153.66 52.74) (end 153.66 54.26) (width 0.5) (layer "B.Cu") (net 42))
 (segment (start 107.5 89) (end 107.5 79) (width 0.5) (layer "B.Cu") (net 22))
 (segment (start 108.08 78.42) (end 111 78.42) (width 0.5) (layer "B.Cu") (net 22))
 (segment (start 108.5 90) (end 107.5 89) (width 0.5) (layer "B.Cu") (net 22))
 (segment (start 118 95.5) (end 118 90) (width 0.5) (layer "B.Cu") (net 22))
 (segment (start 107.5 79) (end 108.08 78.42) (width 0.5) (layer "B.Cu") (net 22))
 (segment (start 154.2 99) (end 121.5 99) (width 0.5) (layer "B.Cu") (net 22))
 (segment (start 118 90) (end 108.5 90) (width 0.5) (layer "B.Cu") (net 22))
 (segment (start 156.2 101) (end 154.2 99) (width 0.5) (layer "B.Cu") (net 22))
 (segment (start 121.5 99) (end 118 95.5) (width 0.5) (layer "B.Cu") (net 22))
 (segment (start 134 85.5) (end 124 85.5) (width 0.5) (layer "B.Cu") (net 5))
 (segment (start 123.5 85) (end 123.5 83.31) (width 0.5) (layer "B.Cu") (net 5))
 (segment (start 124 85.5) (end 123.5 85) (width 0.5) (layer "B.Cu") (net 5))
 (segment (start 141.98 52.74) (end 134 60.72) (width 0.5) (layer "B.Cu") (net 5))
 (segment (start 134 60.72) (end 134 85.5) (width 0.5) (layer "B.Cu") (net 5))
 (segment (start 165.5 100.14) (end 166.36 101) (width 0.5) (layer "F.Cu") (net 15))
 (segment (start 165.5 80.2) (end 165.5 100.14) (width 0.5) (layer "F.Cu") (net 15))
 (segment (start 167 78.7) (end 165.5 80.2) (width 0.5) (layer "F.Cu") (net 15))
 (segment (start 117.5 57.5) (end 117.5 82.5) (width 0.5) (layer "F.Cu") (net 21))
 (segment (start 118 55.5) (end 117.5 56) (width 0.5) (layer "F.Cu") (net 21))
 (segment (start 124.5 89.5) (end 126 89.5) (width 0.5) (layer "F.Cu") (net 21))
 (segment (start 117.5 82.5) (end 124.5 89.5) (width 0.5) (layer "F.Cu") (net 21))
 (segment (start 131.6 55.5) (end 129.5 55.5) (width 0.5) (layer "F.Cu") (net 21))
 (segment (start 134.36 52.74) (end 131.6 55.5) (width 0.5) (layer "F.Cu") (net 21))
 (segment (start 117.5 56) (end 117.5 57.5) (width 0.5) (layer "F.Cu") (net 21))
 (segment (start 129.5 55.5) (end 118 55.5) (width 0.5) (layer "F.Cu") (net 21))
 (via (at 126 89.5) (size 0.8) (drill 0.4) (layers "F.Cu" "B.Cu") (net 21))
 (segment (start 126 89.5) (end 125.92 89.58) (width 0.5) (layer "B.Cu") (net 21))
 (segment (start 125.92 89.58) (end 125.92 95) (width 0.5) (layer "B.Cu") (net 21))
 (segment (start 137.45 54.5) (end 137 54.95) (width 0.5) (layer "F.Cu") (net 7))
 (segment (start 142.76 54.5) (end 137.45 54.5) (width 0.5) (layer "F.Cu") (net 7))
 (segment (start 137 73.81) (end 127.5 83.31) (width 0.5) (layer "F.Cu") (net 7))
 (segment (start 137 54.95) (end 137 73.81) (width 0.5) (layer "F.Cu") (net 7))
 (segment (start 144.52 52.74) (end 142.76 54.5) (width 0.5) (layer "F.Cu") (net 7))
 (segment (start 156.2 52.74) (end 156.2 54.26) (width 0.5) (layer "B.Cu") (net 41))
 (segment (start 156.2 54.26) (end 153.08 57.38) (width 0.5) (layer "B.Cu") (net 41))
 (segment (start 128.08 58.5) (end 133.68 58.5) (width 0.5) (layer "B.Cu") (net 1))
 (segment (start 133.68 58.5) (end 139.44 52.74) (width 0.5) (layer "B.Cu") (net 1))
 (segment (start 167 76.16) (end 164.5 78.66) (width 0.5) (layer "B.Cu") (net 14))
 (segment (start 164.5 100.32) (end 163.82 101) (width 0.5) (layer "B.Cu") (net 14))
 (segment (start 164.5 78.66) (end 164.5 100.32) (width 0.5) (layer "B.Cu") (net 14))
 (segment (start 132.5 57.14) (end 132.5 62) (width 0.5) (layer "F.Cu") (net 20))
 (segment (start 129 88.561508) (end 129.008492 88.57) (width 0.5) (layer "F.Cu") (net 20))
 (segment (start 129 84.5) (end 129 88.561508) (width 0.5) (layer "F.Cu") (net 20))
 (segment (start 136.9 52.74) (end 132.5 57.14) (width 0.5) (layer "F.Cu") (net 20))
 (via (at 129.008492 88.57) (size 0.8) (drill 0.4) (layers "F.Cu" "B.Cu") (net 20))
 (via (at 132.5 62) (size 0.8) (drill 0.4) (layers "F.Cu" "B.Cu") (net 20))
 (via (at 129 84.5) (size 0.8) (drill 0.4) (layers "F.Cu" "B.Cu") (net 20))
 (segment (start 132.5 75.647767) (end 129 79.147767) (width 0.5) (layer "B.Cu") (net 20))
 (segment (start 129.008492 88.57) (end 128.46 89.118492) (width 0.5) (layer "B.Cu") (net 20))
 (segment (start 132.5 62) (end 132.5 75.647767) (width 0.5) (layer "B.Cu") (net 20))
 (segment (start 129 79.147767) (end 129 84.5) (width 0.5) (layer "B.Cu") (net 20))
 (segment (start 128.46 89.118492) (end 128.46 95) (width 0.5) (layer "B.Cu") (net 20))
 (segment (start 167 71.08) (end 162.5 66.58) (width 0.5) (layer "B.Cu") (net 12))
 (segment (start 162.5 55.5) (end 161.5 55.5) (width 0.5) (layer "B.Cu") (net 12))
 (segment (start 162.5 66.58) (end 162.5 55.5) (width 0.5) (layer "B.Cu") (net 12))
 (segment (start 161.5 55.5) (end 158.74 52.74) (width 0.5) (layer "B.Cu") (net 12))
 (segment (start 167 68.54) (end 164 65.54) (width 0.5) (layer "B.Cu") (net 11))
 (segment (start 164 55.46) (end 161.28 52.74) (width 0.5) (layer "B.Cu") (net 11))
 (segment (start 164 65.54) (end 164 55.46) (width 0.5) (layer "B.Cu") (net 11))
 (segment (start 167 54.64) (end 168.9 52.74) (width 0.5) (layer "B.Cu") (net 9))
 (segment (start 167 63.46) (end 167 54.64) (width 0.5) (layer "B.Cu") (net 9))
 (segment (start 145.5 55.5) (end 138 55.5) (width 0.5) (layer "F.Cu") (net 17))
 (segment (start 147.06 53.94) (end 145.5 55.5) (width 0.5) (layer "F.Cu") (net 17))
 (segment (start 138 55.5) (end 138 76) (width 0.5) (layer "F.Cu") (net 17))
 (segment (start 138 76) (end 131 83) (width 0.5) (layer "F.Cu") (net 17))
 (segment (start 147.06 52.74) (end 147.06 53.94) (width 0.5) (layer "F.Cu") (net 17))
 (segment (start 167 66) (end 165.5 64.5) (width 0.5) (layer "B.Cu") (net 10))
 (segment (start 165.5 53.6) (end 166.36 52.74) (width 0.5) (layer "B.Cu") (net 10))
 (segment (start 165.5 64.5) (end 165.5 53.6) (width 0.5) (layer "B.Cu") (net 10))
 (segment (start 163.37 98.91) (end 161.28 101) (width 0.5) (layer "B.Cu") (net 13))
 (segment (start 167 73.62) (end 163.37 77.25) (width 0.5) (layer "B.Cu") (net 13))
 (segment (start 163.37 77.25) (end 163.37 98.91) (width 0.5) (layer "B.Cu") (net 13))
 (segment (start 143.5 101) (end 137.5 95) (width 0.5) (layer "F.Cu") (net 19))
 (segment (start 137.5 95) (end 131 95) (width 0.5) (layer "F.Cu") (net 19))
 (segment (start 131 95) (end 129.7 96.3) (width 0.5) (layer "B.Cu") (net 19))
 (segment (start 137.5 60.26) (end 137.5 88.5) (width 0.5) (layer "B.Cu") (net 19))
 (segment (start 137.5 88.5) (end 131 95) (width 0.5) (layer "B.Cu") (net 19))
 (segment (start 140.38 57.38) (end 137.5 60.26) (width 0.5) (layer "B.Cu") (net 19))
 (segment (start 118.7 89.710051) (end 112.489949 83.5) (width 0.5) (layer "B.Cu") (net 19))
 (segment (start 118.7 92.2) (end 118.7 89.710051) (width 0.5) (layer "B.Cu") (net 19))
 (segment (start 129.7 96.3) (end 122.8 96.3) (width 0.5) (layer "B.Cu") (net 19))
 (segment (start 112.489949 83.5) (end 111 83.5) (width 0.5) (layer "B.Cu") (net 19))
 (segment (start 122.8 96.3) (end 118.7 92.2) (width 0.5) (layer "B.Cu") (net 19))
 (segment (start 150.1 52.74) (end 145.46 57.38) (width 0.5) (layer "B.Cu") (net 43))
 (segment (start 151.12 52.74) (end 150.1 52.74) (width 0.5) (layer "B.Cu") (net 43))
 (segment (start 131.08 66.5) (end 123.5 74.08) (width 0.5) (layer "F.Cu") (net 6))
 (segment (start 123.5 74.08) (end 123.5 75.69) (width 0.5) (layer "F.Cu") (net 6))
 (segment (start 135.5 63) (end 135.5 70) (width 0.5) (layer "F.Cu") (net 8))
 (segment (start 135.5 70) (end 133.19 70) (width 0.5) (layer "F.Cu") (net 8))
 (segment (start 128.5 63) (end 135.5 63) (width 0.5) (layer "F.Cu") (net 8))
 (segment (start 128.54 66.5) (end 128.54 63.04) (width 0.5) (layer "F.Cu") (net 8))
 (segment (start 128.54 63.04) (end 128.5 63) (width 0.25) (layer "F.Cu") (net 8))
 (segment (start 133.19 70) (end 127.5 75.69) (width 0.5) (layer "F.Cu") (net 8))
 (segment (start 131 75.38) (end 131 74.04) (width 0.5) (layer "B.Cu") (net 18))
 (segment (start 131 74.04) (end 123.46 66.5) (width 0.5) (layer "B.Cu") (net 18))
 (segment (start 149.96 70.38) (end 149.96 66.96) (width 0.5) (layer "B.Cu") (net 35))
 (segment (start 149.96 66.96) (end 148 65) (width 0.5) (layer "B.Cu") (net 35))
 (segment (start 147.42 66.96) (end 145.46 65) (width 0.5) (layer "B.Cu") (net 36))
 (segment (start 147.42 70.38) (end 147.42 66.96) (width 0.5) (layer "B.Cu") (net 36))
 (segment (start 142.34 66.96) (end 140.38 65) (width 0.5) (layer "B.Cu") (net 38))
 (segment (start 142.34 70.38) (end 142.34 66.96) (width 0.5) (layer "B.Cu") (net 38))
 (segment (start 157.58 70.38) (end 157.58 66.96) (width 0.5) (layer "B.Cu") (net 32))
 (segment (start 157.58 66.96) (end 155.62 65) (width 0.5) (layer "B.Cu") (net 32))
 (segment (start 152.5 70.38) (end 152.5 66.96) (width 0.5) (layer "B.Cu") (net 34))
 (segment (start 152.5 66.96) (end 150.54 65) (width 0.5) (layer "B.Cu") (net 34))
 (segment (start 144.88 70.38) (end 144.88 66.96) (width 0.5) (layer "B.Cu") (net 37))
 (segment (start 144.88 66.96) (end 142.92 65) (width 0.5) (layer "B.Cu") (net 37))
 (segment (start 155.04 66.96) (end 153.08 65) (width 0.5) (layer "B.Cu") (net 33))
 (segment (start 155.04 70.38) (end 155.04 66.96) (width 0.5) (layer "B.Cu") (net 33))
 (segment (start 158 72.5) (end 142.692233 72.5) (width 0.5) (layer "B.Cu") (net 31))
 (segment (start 142.692233 72.5) (end 138.5 68.307767) (width 0.5) (layer "B.Cu") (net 31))
 (segment (start 160.12 70.38) (end 158 72.5) (width 0.5) (layer "B.Cu") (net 31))
 (segment (start 138.5 68.307767) (end 138.5 61.8) (width 0.5) (layer "B.Cu") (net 31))
 (segment (start 138.5 61.8) (end 142.92 57.38) (width 0.5) (layer "B.Cu") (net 31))
 (segment (start 125.58 58.5) (end 126 58.5) (width 0.25) (layer "F.Cu") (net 2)))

